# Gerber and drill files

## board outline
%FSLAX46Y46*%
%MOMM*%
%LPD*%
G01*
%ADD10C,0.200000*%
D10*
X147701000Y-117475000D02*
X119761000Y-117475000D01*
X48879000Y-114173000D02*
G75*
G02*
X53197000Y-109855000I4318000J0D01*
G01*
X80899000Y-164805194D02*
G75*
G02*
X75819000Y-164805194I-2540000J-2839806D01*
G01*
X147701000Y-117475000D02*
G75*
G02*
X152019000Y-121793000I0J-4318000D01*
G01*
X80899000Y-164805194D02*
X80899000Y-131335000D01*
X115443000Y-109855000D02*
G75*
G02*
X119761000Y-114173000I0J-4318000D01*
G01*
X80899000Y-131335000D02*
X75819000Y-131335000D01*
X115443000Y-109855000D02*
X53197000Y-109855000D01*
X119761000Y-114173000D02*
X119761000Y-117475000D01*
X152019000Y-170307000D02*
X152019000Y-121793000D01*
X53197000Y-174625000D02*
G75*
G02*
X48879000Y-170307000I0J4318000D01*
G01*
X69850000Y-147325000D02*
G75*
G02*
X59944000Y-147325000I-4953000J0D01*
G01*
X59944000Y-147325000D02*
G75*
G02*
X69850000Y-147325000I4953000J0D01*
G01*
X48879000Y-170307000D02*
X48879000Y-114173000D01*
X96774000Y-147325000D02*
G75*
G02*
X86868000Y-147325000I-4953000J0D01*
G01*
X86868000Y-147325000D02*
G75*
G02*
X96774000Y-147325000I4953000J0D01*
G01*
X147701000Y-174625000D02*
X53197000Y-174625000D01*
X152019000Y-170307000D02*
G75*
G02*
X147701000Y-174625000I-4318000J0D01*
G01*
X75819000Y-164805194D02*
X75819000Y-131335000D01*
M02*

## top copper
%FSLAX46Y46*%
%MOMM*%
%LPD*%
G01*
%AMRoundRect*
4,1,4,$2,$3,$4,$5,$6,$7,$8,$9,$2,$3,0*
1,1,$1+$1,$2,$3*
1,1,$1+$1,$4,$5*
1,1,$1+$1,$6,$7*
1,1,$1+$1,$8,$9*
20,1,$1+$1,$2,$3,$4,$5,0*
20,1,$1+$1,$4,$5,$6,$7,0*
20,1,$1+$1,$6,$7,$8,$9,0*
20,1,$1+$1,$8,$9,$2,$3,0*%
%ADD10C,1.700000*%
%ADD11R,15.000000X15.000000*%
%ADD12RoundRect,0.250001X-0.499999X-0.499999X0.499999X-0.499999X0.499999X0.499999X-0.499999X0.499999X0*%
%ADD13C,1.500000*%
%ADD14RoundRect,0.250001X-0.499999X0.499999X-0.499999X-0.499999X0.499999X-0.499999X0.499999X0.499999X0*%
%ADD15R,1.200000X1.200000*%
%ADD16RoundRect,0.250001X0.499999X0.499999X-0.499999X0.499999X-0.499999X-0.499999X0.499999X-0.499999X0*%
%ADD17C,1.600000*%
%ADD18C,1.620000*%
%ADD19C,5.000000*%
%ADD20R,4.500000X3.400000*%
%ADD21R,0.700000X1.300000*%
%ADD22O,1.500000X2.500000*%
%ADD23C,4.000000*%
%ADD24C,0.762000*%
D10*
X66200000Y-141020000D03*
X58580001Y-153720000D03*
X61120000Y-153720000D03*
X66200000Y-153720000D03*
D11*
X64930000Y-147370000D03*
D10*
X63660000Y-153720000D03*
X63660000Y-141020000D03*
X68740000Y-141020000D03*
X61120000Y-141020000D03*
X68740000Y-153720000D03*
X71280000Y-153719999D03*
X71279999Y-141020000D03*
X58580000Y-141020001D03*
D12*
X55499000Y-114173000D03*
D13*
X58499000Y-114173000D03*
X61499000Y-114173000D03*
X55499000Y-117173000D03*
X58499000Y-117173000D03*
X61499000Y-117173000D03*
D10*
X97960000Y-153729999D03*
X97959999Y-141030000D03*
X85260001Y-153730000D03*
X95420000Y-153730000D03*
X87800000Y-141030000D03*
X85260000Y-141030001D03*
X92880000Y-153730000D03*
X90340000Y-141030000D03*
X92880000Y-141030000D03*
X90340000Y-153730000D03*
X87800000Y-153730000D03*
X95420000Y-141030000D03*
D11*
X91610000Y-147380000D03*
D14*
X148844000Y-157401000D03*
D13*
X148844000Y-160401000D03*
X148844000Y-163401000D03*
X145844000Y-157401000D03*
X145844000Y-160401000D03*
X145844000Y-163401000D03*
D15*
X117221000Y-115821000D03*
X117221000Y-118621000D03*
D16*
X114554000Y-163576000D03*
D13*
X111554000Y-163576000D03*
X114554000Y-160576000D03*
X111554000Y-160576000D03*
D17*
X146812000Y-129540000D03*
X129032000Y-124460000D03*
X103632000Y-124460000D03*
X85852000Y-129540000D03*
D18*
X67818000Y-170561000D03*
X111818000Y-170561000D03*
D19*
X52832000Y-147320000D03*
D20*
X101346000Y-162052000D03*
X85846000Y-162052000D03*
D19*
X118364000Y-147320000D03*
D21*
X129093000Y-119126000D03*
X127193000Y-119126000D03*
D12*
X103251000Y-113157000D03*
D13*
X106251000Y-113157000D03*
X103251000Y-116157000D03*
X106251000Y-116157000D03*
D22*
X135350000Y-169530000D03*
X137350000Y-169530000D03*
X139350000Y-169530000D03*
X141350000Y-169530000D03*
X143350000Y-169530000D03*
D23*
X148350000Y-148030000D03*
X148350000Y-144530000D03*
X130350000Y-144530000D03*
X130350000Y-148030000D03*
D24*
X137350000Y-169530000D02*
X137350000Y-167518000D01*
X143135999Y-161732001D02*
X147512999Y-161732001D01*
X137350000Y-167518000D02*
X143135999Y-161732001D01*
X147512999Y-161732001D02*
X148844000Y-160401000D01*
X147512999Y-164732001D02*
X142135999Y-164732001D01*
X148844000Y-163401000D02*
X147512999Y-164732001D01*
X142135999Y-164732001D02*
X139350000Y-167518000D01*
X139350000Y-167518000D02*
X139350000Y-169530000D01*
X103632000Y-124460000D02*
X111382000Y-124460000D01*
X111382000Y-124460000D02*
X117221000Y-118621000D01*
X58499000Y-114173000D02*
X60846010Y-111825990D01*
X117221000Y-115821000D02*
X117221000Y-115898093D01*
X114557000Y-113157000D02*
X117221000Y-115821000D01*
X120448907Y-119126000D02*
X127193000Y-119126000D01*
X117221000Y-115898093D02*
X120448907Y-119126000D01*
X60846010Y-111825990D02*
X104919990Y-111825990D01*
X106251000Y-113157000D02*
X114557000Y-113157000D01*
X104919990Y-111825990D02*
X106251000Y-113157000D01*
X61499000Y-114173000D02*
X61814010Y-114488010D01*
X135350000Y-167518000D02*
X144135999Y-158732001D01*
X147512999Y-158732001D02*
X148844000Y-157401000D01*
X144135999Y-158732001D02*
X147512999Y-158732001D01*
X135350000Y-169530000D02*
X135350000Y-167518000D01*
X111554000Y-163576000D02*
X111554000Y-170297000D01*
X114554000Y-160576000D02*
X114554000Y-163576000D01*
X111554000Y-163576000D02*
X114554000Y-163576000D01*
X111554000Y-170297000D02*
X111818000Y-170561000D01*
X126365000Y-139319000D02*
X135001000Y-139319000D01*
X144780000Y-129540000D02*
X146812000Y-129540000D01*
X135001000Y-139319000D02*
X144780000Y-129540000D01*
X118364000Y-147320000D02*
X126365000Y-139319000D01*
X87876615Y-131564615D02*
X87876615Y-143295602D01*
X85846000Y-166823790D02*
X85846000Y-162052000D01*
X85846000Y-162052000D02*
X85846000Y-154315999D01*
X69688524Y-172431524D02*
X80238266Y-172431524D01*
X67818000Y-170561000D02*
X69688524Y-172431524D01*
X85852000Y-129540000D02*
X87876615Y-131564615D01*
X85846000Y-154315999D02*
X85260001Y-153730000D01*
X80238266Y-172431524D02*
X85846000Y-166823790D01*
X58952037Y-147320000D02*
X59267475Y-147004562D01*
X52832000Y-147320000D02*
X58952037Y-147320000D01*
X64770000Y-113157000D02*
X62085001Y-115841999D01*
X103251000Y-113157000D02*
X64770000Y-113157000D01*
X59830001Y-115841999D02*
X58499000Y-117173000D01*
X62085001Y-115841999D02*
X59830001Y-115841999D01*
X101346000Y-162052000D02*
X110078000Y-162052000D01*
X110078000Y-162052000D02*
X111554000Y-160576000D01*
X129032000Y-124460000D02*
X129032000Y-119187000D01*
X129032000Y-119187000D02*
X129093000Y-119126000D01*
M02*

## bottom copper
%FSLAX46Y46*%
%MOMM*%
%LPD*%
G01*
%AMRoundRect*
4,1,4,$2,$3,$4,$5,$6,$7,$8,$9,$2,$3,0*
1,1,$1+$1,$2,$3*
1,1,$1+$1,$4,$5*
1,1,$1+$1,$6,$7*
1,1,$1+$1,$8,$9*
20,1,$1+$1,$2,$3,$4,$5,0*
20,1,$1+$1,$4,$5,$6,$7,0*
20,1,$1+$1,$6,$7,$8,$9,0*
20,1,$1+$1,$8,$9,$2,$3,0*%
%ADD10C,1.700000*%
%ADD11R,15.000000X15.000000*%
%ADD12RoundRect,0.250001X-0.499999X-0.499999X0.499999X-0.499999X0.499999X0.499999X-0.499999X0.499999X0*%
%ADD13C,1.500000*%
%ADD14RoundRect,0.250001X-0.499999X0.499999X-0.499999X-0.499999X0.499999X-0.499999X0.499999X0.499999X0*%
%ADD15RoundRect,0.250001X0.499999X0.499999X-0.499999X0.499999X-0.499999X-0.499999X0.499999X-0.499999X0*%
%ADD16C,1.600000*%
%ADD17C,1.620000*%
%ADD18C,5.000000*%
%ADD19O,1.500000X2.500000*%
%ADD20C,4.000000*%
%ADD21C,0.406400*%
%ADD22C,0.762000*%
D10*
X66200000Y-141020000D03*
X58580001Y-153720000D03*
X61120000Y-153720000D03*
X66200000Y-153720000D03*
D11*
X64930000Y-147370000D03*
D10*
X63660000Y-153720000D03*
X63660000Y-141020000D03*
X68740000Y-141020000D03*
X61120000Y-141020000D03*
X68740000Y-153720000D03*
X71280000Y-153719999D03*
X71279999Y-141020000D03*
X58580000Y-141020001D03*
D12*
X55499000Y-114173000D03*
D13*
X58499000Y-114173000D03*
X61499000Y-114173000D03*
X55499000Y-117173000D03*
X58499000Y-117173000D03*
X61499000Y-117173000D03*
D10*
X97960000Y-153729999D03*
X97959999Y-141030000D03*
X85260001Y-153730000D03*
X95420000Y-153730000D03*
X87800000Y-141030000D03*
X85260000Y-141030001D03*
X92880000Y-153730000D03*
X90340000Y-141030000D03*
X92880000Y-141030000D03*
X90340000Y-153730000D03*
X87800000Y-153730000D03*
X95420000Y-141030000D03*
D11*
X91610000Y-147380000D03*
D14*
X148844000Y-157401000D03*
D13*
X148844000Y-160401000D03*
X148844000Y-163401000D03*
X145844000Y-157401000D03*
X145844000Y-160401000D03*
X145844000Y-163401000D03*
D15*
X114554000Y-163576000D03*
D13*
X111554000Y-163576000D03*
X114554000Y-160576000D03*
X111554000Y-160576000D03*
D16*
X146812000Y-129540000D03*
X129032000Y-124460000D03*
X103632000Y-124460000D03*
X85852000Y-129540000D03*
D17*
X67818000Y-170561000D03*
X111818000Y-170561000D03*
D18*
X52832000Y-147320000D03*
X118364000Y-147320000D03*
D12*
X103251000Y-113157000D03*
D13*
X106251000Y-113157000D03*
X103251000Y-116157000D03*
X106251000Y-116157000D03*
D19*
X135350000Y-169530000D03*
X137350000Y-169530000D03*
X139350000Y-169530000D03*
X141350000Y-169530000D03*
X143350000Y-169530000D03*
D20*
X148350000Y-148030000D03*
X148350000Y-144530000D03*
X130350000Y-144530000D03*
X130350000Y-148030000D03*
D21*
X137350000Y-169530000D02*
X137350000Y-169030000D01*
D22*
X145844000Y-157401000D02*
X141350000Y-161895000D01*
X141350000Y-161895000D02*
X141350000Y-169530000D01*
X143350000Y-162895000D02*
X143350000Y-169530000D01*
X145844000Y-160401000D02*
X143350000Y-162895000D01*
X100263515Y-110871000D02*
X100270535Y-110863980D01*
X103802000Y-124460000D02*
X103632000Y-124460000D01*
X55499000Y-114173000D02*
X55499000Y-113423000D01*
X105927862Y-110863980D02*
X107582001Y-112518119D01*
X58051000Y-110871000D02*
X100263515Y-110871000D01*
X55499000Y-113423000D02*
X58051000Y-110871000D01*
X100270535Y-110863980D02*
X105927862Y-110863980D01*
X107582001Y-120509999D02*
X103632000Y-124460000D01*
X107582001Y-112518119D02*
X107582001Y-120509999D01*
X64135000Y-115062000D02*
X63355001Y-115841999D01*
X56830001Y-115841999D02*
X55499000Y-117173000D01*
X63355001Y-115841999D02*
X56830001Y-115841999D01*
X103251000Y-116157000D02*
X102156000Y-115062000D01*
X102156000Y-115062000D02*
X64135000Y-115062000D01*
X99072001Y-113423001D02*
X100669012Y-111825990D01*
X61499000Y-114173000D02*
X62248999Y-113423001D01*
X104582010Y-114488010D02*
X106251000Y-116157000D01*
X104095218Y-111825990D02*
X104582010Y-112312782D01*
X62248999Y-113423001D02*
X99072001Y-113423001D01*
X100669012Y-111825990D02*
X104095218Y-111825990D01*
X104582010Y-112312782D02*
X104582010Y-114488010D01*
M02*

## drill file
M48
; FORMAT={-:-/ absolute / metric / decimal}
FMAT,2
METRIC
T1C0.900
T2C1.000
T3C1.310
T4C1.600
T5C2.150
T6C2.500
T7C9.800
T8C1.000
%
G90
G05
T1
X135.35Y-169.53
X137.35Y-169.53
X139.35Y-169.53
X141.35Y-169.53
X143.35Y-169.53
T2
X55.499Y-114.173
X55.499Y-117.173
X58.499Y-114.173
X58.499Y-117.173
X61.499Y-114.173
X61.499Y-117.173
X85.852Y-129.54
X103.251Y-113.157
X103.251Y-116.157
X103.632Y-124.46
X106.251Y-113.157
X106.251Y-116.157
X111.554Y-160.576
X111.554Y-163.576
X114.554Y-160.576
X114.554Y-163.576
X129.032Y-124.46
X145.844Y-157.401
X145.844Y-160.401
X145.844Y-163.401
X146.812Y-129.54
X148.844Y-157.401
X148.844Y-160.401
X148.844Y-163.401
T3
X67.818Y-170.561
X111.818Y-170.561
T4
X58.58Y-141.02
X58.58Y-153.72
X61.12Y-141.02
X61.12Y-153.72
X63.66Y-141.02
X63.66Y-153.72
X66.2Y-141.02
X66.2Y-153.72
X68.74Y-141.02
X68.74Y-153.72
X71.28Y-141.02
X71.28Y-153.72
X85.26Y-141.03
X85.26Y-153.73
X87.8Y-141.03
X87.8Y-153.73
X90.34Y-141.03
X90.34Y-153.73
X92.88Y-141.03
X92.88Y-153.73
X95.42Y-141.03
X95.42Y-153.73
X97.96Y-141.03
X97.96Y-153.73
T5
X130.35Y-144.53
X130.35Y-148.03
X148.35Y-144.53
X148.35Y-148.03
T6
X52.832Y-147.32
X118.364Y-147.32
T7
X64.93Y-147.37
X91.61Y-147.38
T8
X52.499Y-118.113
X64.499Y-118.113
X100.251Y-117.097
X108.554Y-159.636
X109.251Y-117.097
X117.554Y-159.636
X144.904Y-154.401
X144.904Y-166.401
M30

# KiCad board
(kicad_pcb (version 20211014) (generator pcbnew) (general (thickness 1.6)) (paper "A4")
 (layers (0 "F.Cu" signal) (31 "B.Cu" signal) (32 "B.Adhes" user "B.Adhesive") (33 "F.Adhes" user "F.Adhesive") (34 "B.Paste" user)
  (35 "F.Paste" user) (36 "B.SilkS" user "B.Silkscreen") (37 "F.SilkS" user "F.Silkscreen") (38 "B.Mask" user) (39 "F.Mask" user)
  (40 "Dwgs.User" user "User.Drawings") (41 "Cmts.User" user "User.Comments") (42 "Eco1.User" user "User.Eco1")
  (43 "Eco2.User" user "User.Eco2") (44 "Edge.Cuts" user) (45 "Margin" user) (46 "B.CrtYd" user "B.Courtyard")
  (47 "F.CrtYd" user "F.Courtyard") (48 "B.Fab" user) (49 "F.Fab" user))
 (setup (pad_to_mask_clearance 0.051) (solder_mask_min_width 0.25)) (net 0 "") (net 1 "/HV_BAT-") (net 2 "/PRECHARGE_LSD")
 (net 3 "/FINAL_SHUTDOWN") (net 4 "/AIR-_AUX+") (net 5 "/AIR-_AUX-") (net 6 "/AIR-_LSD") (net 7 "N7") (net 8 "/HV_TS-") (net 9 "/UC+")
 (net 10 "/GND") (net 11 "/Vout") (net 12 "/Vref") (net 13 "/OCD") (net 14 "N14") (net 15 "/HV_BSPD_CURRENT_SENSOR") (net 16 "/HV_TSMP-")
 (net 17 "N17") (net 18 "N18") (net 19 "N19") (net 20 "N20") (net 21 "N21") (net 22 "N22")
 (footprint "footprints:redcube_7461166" (layer "F.Cu") (at 64.93 147.37)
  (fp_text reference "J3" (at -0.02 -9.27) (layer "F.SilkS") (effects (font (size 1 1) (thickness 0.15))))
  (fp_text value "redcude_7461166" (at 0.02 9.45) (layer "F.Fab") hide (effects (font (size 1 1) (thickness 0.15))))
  (pad "1" thru_hole circle locked (at 1.27 -6.35) (size 1.7 1.7) (drill 1.6) (layers *.Cu *.Mask) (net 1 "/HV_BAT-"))
  (pad "1" thru_hole circle locked (at -6.349999 6.35) (size 1.7 1.7) (drill 1.6) (layers *.Cu *.Mask) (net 1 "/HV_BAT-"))
  (pad "1" thru_hole circle locked (at -3.81 6.35) (size 1.7 1.7) (drill 1.6) (layers *.Cu *.Mask) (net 1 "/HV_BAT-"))
  (pad "1" thru_hole circle locked (at 1.27 6.35) (size 1.7 1.7) (drill 1.6) (layers *.Cu *.Mask) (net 1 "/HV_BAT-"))
  (pad "1" thru_hole rect locked (at 0 0) (size 15 15) (drill 9.8) (layers *.Cu *.Mask) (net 1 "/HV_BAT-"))
  (pad "1" thru_hole circle locked (at -1.27 6.35) (size 1.7 1.7) (drill 1.6) (layers *.Cu *.Mask) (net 1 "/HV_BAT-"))
  (pad "1" thru_hole circle locked (at -1.27 -6.35) (size 1.7 1.7) (drill 1.6) (layers *.Cu *.Mask) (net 1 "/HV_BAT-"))
  (pad "1" thru_hole circle locked (at 3.81 -6.35) (size 1.7 1.7) (drill 1.6) (layers *.Cu *.Mask) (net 1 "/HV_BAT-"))
  (pad "1" thru_hole circle locked (at -3.81 -6.35) (size 1.7 1.7) (drill 1.6) (layers *.Cu *.Mask) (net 1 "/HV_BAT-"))
  (pad "1" thru_hole circle locked (at 3.81 6.35) (size 1.7 1.7) (drill 1.6) (layers *.Cu *.Mask) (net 1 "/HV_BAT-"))
  (pad "1" thru_hole circle locked (at 6.35 6.349999) (size 1.7 1.7) (drill 1.6) (layers *.Cu *.Mask) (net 1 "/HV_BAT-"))
  (pad "1" thru_hole circle locked (at 6.349999 -6.35) (size 1.7 1.7) (drill 1.6) (layers *.Cu *.Mask) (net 1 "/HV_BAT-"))
  (pad "1" thru_hole circle locked (at -6.35 -6.349999) (size 1.7 1.7) (drill 1.6) (layers *.Cu *.Mask) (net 1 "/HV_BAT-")))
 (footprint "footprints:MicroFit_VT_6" (layer "F.Cu") (at 55.499 114.173)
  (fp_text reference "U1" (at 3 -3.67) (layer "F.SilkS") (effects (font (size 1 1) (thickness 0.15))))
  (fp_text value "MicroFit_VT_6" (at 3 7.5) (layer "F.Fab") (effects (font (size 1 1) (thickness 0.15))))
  (pad "" np_thru_hole circle locked (at -3 3.94) (size 1 1) (drill 1) (layers *.Cu *.Mask))
  (pad "" np_thru_hole circle locked (at 9 3.94) (size 1 1) (drill 1) (layers *.Cu *.Mask))
  (pad "1" thru_hole roundrect locked (at 0 0) (size 1.5 1.5) (drill 1) (layers *.Cu *.Mask) (roundrect_rratio 0.166667)
   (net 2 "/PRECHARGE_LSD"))
  (pad "2" thru_hole circle locked (at 3 0) (size 1.5 1.5) (drill 1) (layers *.Cu *.Mask) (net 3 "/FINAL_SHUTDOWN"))
  (pad "3" thru_hole circle locked (at 6 0) (size 1.5 1.5) (drill 1) (layers *.Cu *.Mask) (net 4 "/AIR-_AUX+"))
  (pad "4" thru_hole circle locked (at 0 3) (size 1.5 1.5) (drill 1) (layers *.Cu *.Mask) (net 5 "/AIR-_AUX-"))
  (pad "5" thru_hole circle locked (at 3 3) (size 1.5 1.5) (drill 1) (layers *.Cu *.Mask) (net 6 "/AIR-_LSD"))
  (pad "6" thru_hole circle locked (at 6 3) (size 1.5 1.5) (drill 1) (layers *.Cu *.Mask) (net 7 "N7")))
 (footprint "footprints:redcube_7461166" (layer "F.Cu") (at 91.61 147.38)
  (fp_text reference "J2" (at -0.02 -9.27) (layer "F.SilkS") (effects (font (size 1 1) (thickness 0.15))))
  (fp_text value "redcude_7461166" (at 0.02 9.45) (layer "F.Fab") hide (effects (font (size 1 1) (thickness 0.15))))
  (pad "1" thru_hole circle locked (at 6.35 6.349999) (size 1.7 1.7) (drill 1.6) (layers *.Cu *.Mask) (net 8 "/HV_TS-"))
  (pad "1" thru_hole circle locked (at 6.349999 -6.35) (size 1.7 1.7) (drill 1.6) (layers *.Cu *.Mask) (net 8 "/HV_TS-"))
  (pad "1" thru_hole circle locked (at -6.349999 6.35) (size 1.7 1.7) (drill 1.6) (layers *.Cu *.Mask) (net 8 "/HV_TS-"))
  (pad "1" thru_hole circle locked (at 3.81 6.35) (size 1.7 1.7) (drill 1.6) (layers *.Cu *.Mask) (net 8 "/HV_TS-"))
  (pad "1" thru_hole circle locked (at -3.81 -6.35) (size 1.7 1.7) (drill 1.6) (layers *.Cu *.Mask) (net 8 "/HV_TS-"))
  (pad "1" thru_hole circle locked (at -6.35 -6.349999) (size 1.7 1.7) (drill 1.6) (layers *.Cu *.Mask) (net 8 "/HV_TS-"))
  (pad "1" thru_hole circle locked (at 1.27 6.35) (size 1.7 1.7) (drill 1.6) (layers *.Cu *.Mask) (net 8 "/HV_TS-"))
  (pad "1" thru_hole circle locked (at -1.27 -6.35) (size 1.7 1.7) (drill 1.6) (layers *.Cu *.Mask) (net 8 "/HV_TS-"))
  (pad "1" thru_hole circle locked (at 1.27 -6.35) (size 1.7 1.7) (drill 1.6) (layers *.Cu *.Mask) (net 8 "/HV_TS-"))
  (pad "1" thru_hole circle locked (at -1.27 6.35) (size 1.7 1.7) (drill 1.6) (layers *.Cu *.Mask) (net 8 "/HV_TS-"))
  (pad "1" thru_hole circle locked (at -3.81 6.35) (size 1.7 1.7) (drill 1.6) (layers *.Cu *.Mask) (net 8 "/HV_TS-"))
  (pad "1" thru_hole circle locked (at 3.81 -6.35) (size 1.7 1.7) (drill 1.6) (layers *.Cu *.Mask) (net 8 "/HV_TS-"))
  (pad "1" thru_hole rect locked (at 0 0) (size 15 15) (drill 9.8) (layers *.Cu *.Mask) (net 8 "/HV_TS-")))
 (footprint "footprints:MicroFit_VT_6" (layer "F.Cu") (at 148.844 157.401 -90)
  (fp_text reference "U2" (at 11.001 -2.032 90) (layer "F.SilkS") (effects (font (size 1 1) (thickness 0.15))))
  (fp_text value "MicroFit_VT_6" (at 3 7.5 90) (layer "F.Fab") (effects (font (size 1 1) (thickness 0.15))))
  (pad "" np_thru_hole circle locked (at 9 3.94 270) (size 1 1) (drill 1) (layers *.Cu *.Mask))
  (pad "" np_thru_hole circle locked (at -3 3.94 270) (size 1 1) (drill 1) (layers *.Cu *.Mask))
  (pad "1" thru_hole roundrect locked (at 0 0 270) (size 1.5 1.5) (drill 1) (layers *.Cu *.Mask) (roundrect_rratio 0.166667) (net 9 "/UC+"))
  (pad "2" thru_hole circle locked (at 3 0 270) (size 1.5 1.5) (drill 1) (layers *.Cu *.Mask) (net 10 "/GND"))
  (pad "3" thru_hole circle locked (at 6 0 270) (size 1.5 1.5) (drill 1) (layers *.Cu *.Mask) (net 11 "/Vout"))
  (pad "4" thru_hole circle locked (at 0 3 270) (size 1.5 1.5) (drill 1) (layers *.Cu *.Mask) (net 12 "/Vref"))
  (pad "5" thru_hole circle locked (at 3 3 270) (size 1.5 1.5) (drill 1) (layers *.Cu *.Mask) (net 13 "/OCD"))
  (pad "6" thru_hole circle locked (at 6 3 270) (size 1.5 1.5) (drill 1) (layers *.Cu *.Mask) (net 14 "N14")))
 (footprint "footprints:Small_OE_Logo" (layer "F.Cu") (at 60.071 127)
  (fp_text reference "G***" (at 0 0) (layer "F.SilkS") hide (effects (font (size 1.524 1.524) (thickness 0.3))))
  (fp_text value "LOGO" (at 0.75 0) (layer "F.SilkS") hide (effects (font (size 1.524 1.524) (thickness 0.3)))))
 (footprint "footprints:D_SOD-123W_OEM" (layer "F.Cu") (at 117.221 117.221 -90)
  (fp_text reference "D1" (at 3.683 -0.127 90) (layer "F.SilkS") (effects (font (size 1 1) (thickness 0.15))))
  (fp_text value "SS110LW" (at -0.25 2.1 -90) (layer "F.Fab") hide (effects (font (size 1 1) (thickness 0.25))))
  (pad "1" smd rect locked (at -1.4 0 270) (size 1.2 1.2) (layers "F.Cu" "F.Paste" "F.Mask") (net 3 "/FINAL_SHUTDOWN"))
  (pad "2" smd rect locked (at 1.4 0 270) (size 1.2 1.2) (layers "F.Cu" "F.Paste" "F.Mask") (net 2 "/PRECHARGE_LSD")))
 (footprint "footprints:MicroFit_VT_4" (layer "F.Cu") (at 114.554 163.576 180)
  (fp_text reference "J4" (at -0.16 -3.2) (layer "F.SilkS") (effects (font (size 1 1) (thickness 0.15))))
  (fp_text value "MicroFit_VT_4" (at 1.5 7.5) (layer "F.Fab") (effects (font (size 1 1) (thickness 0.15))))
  (pad "" np_thru_hole circle locked (at -3 3.94 180) (size 1 1) (drill 1) (layers *.Cu *.Mask))
  (pad "" np_thru_hole circle locked (at 6 3.94 180) (size 1 1) (drill 1) (layers *.Cu *.Mask))
  (pad "1" thru_hole roundrect locked (at 0 0 180) (size 1.5 1.5) (drill 1) (layers *.Cu *.Mask) (roundrect_rratio 0.166667)
   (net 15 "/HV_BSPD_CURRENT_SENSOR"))
  (pad "2" thru_hole circle locked (at 3 0 180) (size 1.5 1.5) (drill 1) (layers *.Cu *.Mask) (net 15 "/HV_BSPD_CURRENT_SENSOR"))
  (pad "3" thru_hole circle locked (at 0 3 180) (size 1.5 1.5) (drill 1) (layers *.Cu *.Mask) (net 15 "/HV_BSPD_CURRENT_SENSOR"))
  (pad "4" thru_hole circle locked (at 3 3 180) (size 1.5 1.5) (drill 1) (layers *.Cu *.Mask) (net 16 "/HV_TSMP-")))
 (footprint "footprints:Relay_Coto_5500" (layer "F.Cu") (at 82.042 137.033)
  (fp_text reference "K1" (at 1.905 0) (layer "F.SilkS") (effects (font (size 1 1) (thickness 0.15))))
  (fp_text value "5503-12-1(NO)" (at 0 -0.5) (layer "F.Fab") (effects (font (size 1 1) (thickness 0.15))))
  (pad "1" thru_hole circle locked (at 64.77 -7.493) (size 1.6 1.6) (drill 1) (layers *.Cu *.Mask) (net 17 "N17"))
  (pad "2" thru_hole circle locked (at 46.99 -12.573) (size 1.6 1.6) (drill 1) (layers *.Cu *.Mask) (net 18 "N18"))
  (pad "3" thru_hole circle locked (at 21.59 -12.573) (size 1.6 1.6) (drill 1) (layers *.Cu *.Mask) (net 2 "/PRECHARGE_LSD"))
  (pad "4" thru_hole circle locked (at 3.81 -7.493) (size 1.6 1.6) (drill 1) (layers *.Cu *.Mask) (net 8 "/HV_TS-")))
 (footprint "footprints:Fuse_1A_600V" (layer "F.Cu") (at 67.818 170.561)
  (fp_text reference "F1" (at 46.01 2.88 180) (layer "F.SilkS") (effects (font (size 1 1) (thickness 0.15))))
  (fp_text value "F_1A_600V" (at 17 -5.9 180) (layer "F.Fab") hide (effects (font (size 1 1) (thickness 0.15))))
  (pad "1" thru_hole circle locked (at 0 0) (size 1.62 1.62) (drill 1.31) (layers *.Cu *.Mask) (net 8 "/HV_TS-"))
  (pad "2" thru_hole circle locked (at 44 0) (size 1.62 1.62) (drill 1.31) (layers *.Cu *.Mask) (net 15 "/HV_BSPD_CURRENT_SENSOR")))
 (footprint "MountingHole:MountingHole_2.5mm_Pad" (layer "F.Cu") (at 52.832 147.32)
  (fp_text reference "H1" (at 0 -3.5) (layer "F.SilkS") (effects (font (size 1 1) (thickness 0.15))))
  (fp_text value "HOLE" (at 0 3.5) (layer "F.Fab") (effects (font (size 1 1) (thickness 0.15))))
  (pad "1" thru_hole circle locked (at 0 0) (size 5 5) (drill 2.5) (layers *.Cu *.Mask) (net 1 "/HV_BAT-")))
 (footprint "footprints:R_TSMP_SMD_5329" (layer "F.Cu") (at 93.726 162.052 180)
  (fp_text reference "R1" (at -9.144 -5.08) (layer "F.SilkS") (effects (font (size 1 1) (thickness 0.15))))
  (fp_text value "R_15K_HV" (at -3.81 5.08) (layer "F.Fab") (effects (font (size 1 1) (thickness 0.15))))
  (pad "1" smd rect locked (at -7.62 0 180) (size 4.5 3.4) (layers "F.Cu" "F.Paste" "F.Mask") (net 16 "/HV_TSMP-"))
  (pad "2" smd rect locked (at 7.88 0 180) (size 4.5 3.4) (layers "F.Cu" "F.Paste" "F.Mask") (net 8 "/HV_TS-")))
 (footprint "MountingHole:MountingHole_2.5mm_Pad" (layer "F.Cu") (at 118.364 147.32)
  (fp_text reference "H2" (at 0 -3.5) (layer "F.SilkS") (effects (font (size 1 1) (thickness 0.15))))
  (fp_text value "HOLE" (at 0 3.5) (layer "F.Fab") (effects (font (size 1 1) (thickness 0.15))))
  (pad "1" thru_hole circle locked (at 0 0) (size 5 5) (drill 2.5) (layers *.Cu *.Mask) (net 17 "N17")))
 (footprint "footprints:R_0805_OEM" (layer "F.Cu") (at 128.143 119.126 180)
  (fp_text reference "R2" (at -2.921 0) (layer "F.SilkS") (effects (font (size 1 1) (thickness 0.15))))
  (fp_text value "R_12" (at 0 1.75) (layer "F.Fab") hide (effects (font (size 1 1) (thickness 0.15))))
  (pad "1" smd rect locked (at -0.95 0 180) (size 0.7 1.3) (layers "F.Cu" "F.Paste" "F.Mask") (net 18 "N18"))
  (pad "2" smd rect locked (at 0.95 0 180) (size 0.7 1.3) (layers "F.Cu" "F.Paste" "F.Mask") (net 3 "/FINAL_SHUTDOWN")))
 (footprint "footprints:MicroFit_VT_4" (layer "F.Cu") (at 103.251 113.157)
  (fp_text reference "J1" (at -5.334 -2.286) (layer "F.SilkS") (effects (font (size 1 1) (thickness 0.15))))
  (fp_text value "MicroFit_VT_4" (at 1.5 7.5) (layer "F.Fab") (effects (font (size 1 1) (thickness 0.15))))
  (pad "" np_thru_hole circle locked (at 6 3.94) (size 1 1) (drill 1) (layers *.Cu *.Mask))
  (pad "" np_thru_hole circle locked (at -3 3.94) (size 1 1) (drill 1) (layers *.Cu *.Mask))
  (pad "1" thru_hole roundrect locked (at 0 0) (size 1.5 1.5) (drill 1) (layers *.Cu *.Mask) (roundrect_rratio 0.166667) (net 6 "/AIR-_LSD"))
  (pad "2" thru_hole circle locked (at 3 0) (size 1.5 1.5) (drill 1) (layers *.Cu *.Mask) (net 3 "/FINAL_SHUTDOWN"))
  (pad "3" thru_hole circle locked (at 0 3) (size 1.5 1.5) (drill 1) (layers *.Cu *.Mask) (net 5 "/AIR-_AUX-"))
  (pad "4" thru_hole circle locked (at 3 3) (size 1.5 1.5) (drill 1) (layers *.Cu *.Mask) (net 4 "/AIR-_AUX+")))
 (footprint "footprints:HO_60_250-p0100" (layer "B.Cu") (at 130.35 144.53 -90)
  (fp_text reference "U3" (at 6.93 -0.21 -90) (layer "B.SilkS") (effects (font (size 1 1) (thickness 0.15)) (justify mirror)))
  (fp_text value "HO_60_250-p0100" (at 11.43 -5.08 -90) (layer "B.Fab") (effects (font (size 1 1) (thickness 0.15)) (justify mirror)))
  (pad "1" thru_hole oval locked (at 25 -5 270) (size 2.5 1.5) (drill 0.9) (layers *.Cu *.Mask) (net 9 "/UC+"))
  (pad "2" thru_hole oval locked (at 25 -7 270) (size 2.5 1.5) (drill 0.9) (layers *.Cu *.Mask) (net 10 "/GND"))
  (pad "3" thru_hole oval locked (at 25 -9 270) (size 2.5 1.5) (drill 0.9) (layers *.Cu *.Mask) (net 11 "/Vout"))
  (pad "4" thru_hole oval locked (at 25 -11 270) (size 2.5 1.5) (drill 0.9) (layers *.Cu *.Mask) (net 12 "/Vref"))
  (pad "5" thru_hole oval locked (at 25 -13 270) (size 2.5 1.5) (drill 0.9) (layers *.Cu *.Mask) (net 13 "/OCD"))
  (pad "7" thru_hole circle locked (at 3.5 -18 270) (size 4 4) (drill 2.15) (layers *.Cu *.Mask) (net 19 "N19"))
  (pad "8" thru_hole circle locked (at 0 -18 270) (size 4 4) (drill 2.15) (layers *.Cu *.Mask) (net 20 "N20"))
  (pad "11" thru_hole circle locked (at 0 0 270) (size 4 4) (drill 2.15) (layers *.Cu *.Mask) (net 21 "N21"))
  (pad "12" thru_hole circle locked (at 3.5 0 270) (size 4 4) (drill 2.15) (layers *.Cu *.Mask) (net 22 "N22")))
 (gr_line (start 147.701 117.475) (end 119.761 117.475) (layer "Edge.Cuts") (width 0.2))
 (gr_arc (start 48.879 114.173) (mid 50.143713 111.119713) (end 53.197 109.855) (layer "Edge.Cuts") (width 0.2))
 (gr_arc (start 80.899 164.805194) (mid 78.359 171.455) (end 75.819 164.805194) (layer "Edge.Cuts") (width 0.2))
 (gr_arc (start 147.701 117.475) (mid 150.754287 118.739713) (end 152.019 121.793) (layer "Edge.Cuts") (width 0.2))
 (gr_line (start 80.899 164.805194) (end 80.899 131.335) (layer "Edge.Cuts") (width 0.2))
 (gr_arc (start 115.443 109.855) (mid 118.496287 111.119713) (end 119.761 114.173) (layer "Edge.Cuts") (width 0.2))
 (gr_line (start 80.899 131.335) (end 75.819 131.335) (layer "Edge.Cuts") (width 0.2))
 (gr_line (start 115.443 109.855) (end 53.197 109.855) (layer "Edge.Cuts") (width 0.2))
 (gr_line (start 119.761 114.173) (end 119.761 117.475) (layer "Edge.Cuts") (width 0.2))
 (gr_line (start 152.019 170.307) (end 152.019 121.793) (layer "Edge.Cuts") (width 0.2))
 (gr_arc (start 53.197 174.625) (mid 50.143713 173.360287) (end 48.879 170.307) (layer "Edge.Cuts") (width 0.2))
 (gr_circle (center 64.897 147.325) (end 59.944 147.325) (layer "Edge.Cuts") (width 0.2) (fill none))
 (gr_line (start 48.879 170.307) (end 48.879 114.173) (layer "Edge.Cuts") (width 0.2))
 (gr_circle (center 91.821 147.325) (end 86.868 147.325) (layer "Edge.Cuts") (width 0.2) (fill none))
 (gr_line (start 147.701 174.625) (end 53.197 174.625) (layer "Edge.Cuts") (width 0.2))
 (gr_arc (start 152.019 170.307) (mid 150.754287 173.360287) (end 147.701 174.625) (layer "Edge.Cuts") (width 0.2))
 (gr_line (start 75.819 164.805194) (end 75.819 131.335) (layer "Edge.Cuts") (width 0.2))
 (segment (start 137.35 169.53) (end 137.35 167.518) (width 0.762) (layer "F.Cu") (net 10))
 (segment (start 143.135999 161.732001) (end 147.512999 161.732001) (width 0.762) (layer "F.Cu") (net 10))
 (segment (start 137.35 167.518) (end 143.135999 161.732001) (width 0.762) (layer "F.Cu") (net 10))
 (segment (start 147.512999 161.732001) (end 148.844 160.401) (width 0.762) (layer "F.Cu") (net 10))
 (segment (start 137.35 169.53) (end 137.35 169.03) (width 0.4064) (layer "B.Cu") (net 10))
 (segment (start 147.512999 164.732001) (end 142.135999 164.732001) (width 0.762) (layer "F.Cu") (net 11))
 (segment (start 148.844 163.401) (end 147.512999 164.732001) (width 0.762) (layer "F.Cu") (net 11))
 (segment (start 142.135999 164.732001) (end 139.35 167.518) (width 0.762) (layer "F.Cu") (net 11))
 (segment (start 139.35 167.518) (end 139.35 169.53) (width 0.762) (layer "F.Cu") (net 11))
 (segment (start 145.844 157.401) (end 141.35 161.895) (width 0.762) (layer "B.Cu") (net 12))
 (segment (start 141.35 161.895) (end 141.35 169.53) (width 0.762) (layer "B.Cu") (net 12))
 (segment (start 143.35 162.895) (end 143.35 169.53) (width 0.762) (layer "B.Cu") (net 13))
 (segment (start 145.844 160.401) (end 143.35 162.895) (width 0.762) (layer "B.Cu") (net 13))
 (segment (start 103.632 124.46) (end 111.382 124.46) (width 0.762) (layer "F.Cu") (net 2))
 (segment (start 111.382 124.46) (end 117.221 118.621) (width 0.762) (layer "F.Cu") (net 2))
 (segment (start 100.263515 110.871) (end 100.270535 110.86398) (width 0.762) (layer "B.Cu") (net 2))
 (segment (start 103.802 124.46) (end 103.632 124.46) (width 0.762) (layer "B.Cu") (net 2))
 (segment (start 55.499 114.173) (end 55.499 113.423) (width 0.762) (layer "B.Cu") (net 2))
 (segment (start 105.927862 110.86398) (end 107.582001 112.518119) (width 0.762) (layer "B.Cu") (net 2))
 (segment (start 58.051 110.871) (end 100.263515 110.871) (width 0.762) (layer "B.Cu") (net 2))
 (segment (start 55.499 113.423) (end 58.051 110.871) (width 0.762) (layer "B.Cu") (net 2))
 (segment (start 100.270535 110.86398) (end 105.927862 110.86398) (width 0.762) (layer "B.Cu") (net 2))
 (segment (start 107.582001 120.509999) (end 103.632 124.46) (width 0.762) (layer "B.Cu") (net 2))
 (segment (start 107.582001 112.518119) (end 107.582001 120.509999) (width 0.762) (layer "B.Cu") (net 2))
 (segment (start 58.499 114.173) (end 60.84601 111.82599) (width 0.762) (layer "F.Cu") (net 3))
 (segment (start 117.221 115.821) (end 117.221 115.898093) (width 0.762) (layer "F.Cu") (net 3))
 (segment (start 114.557 113.157) (end 117.221 115.821) (width 0.762) (layer "F.Cu") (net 3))
 (segment (start 120.448907 119.126) (end 127.193 119.126) (width 0.762) (layer "F.Cu") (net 3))
 (segment (start 117.221 115.898093) (end 120.448907 119.126) (width 0.762) (layer "F.Cu") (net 3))
 (segment (start 60.84601 111.82599) (end 104.91999 111.82599) (width 0.762) (layer "F.Cu") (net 3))
 (segment (start 106.251 113.157) (end 114.557 113.157) (width 0.762) (layer "F.Cu") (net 3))
 (segment (start 104.91999 111.82599) (end 106.251 113.157) (width 0.762) (layer "F.Cu") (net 3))
 (segment (start 64.135 115.062) (end 63.355001 115.841999) (width 0.762) (layer "B.Cu") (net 5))
 (segment (start 56.830001 115.841999) (end 55.499 117.173) (width 0.762) (layer "B.Cu") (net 5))
 (segment (start 63.355001 115.841999) (end 56.830001 115.841999) (width 0.762) (layer "B.Cu") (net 5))
 (segment (start 103.251 116.157) (end 102.156 115.062) (width 0.762) (layer "B.Cu") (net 5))
 (segment (start 102.156 115.062) (end 64.135 115.062) (width 0.762) (layer "B.Cu") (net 5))
 (segment (start 61.499 114.173) (end 61.81401 114.48801) (width 0.762) (layer "F.Cu") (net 4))
 (segment (start 99.072001 113.423001) (end 100.669012 111.82599) (width 0.762) (layer "B.Cu") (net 4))
 (segment (start 61.499 114.173) (end 62.248999 113.423001) (width 0.762) (layer "B.Cu") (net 4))
 (segment (start 104.58201 114.48801) (end 106.251 116.157) (width 0.762) (layer "B.Cu") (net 4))
 (segment (start 104.095218 111.82599) (end 104.58201 112.312782) (width 0.762) (layer "B.Cu") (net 4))
 (segment (start 62.248999 113.423001) (end 99.072001 113.423001) (width 0.762) (layer "B.Cu") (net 4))
 (segment (start 100.669012 111.82599) (end 104.095218 111.82599) (width 0.762) (layer "B.Cu") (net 4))
 (segment (start 104.58201 112.312782) (end 104.58201 114.48801) (width 0.762) (layer "B.Cu") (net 4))
 (segment (start 135.35 167.518) (end 144.135999 158.732001) (width 0.762) (layer "F.Cu") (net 9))
 (segment (start 147.512999 158.732001) (end 148.844 157.401) (width 0.762) (layer "F.Cu") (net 9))
 (segment (start 144.135999 158.732001) (end 147.512999 158.732001) (width 0.762) (layer "F.Cu") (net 9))
 (segment (start 135.35 169.53) (end 135.35 167.518) (width 0.762) (layer "F.Cu") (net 9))
 (segment (start 111.554 163.576) (end 111.554 170.297) (width 0.762) (layer "F.Cu") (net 15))
 (segment (start 114.554 160.576) (end 114.554 163.576) (width 0.762) (layer "F.Cu") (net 15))
 (segment (start 111.554 163.576) (end 114.554 163.576) (width 0.762) (layer "F.Cu") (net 15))
 (segment (start 111.554 170.297) (end 111.818 170.561) (width 0.762) (layer "F.Cu") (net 15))
 (segment (start 126.365 139.319) (end 135.001 139.319) (width 0.762) (layer "F.Cu") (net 17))
 (segment (start 144.78 129.54) (end 146.812 129.54) (width 0.762) (layer "F.Cu") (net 17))
 (segment (start 135.001 139.319) (end 144.78 129.54) (width 0.762) (layer "F.Cu") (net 17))
 (segment (start 118.364 147.32) (end 126.365 139.319) (width 0.762) (layer "F.Cu") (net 17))
 (segment (start 87.876615 131.564615) (end 87.876615 143.295602) (width 0.762) (layer "F.Cu") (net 8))
 (segment (start 85.846 166.82379) (end 85.846 162.052) (width 0.762) (layer "F.Cu") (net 8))
 (segment (start 85.846 162.052) (end 85.846 154.315999) (width 0.762) (layer "F.Cu") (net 8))
 (segment (start 69.688524 172.431524) (end 80.238266 172.431524) (width 0.762) (layer "F.Cu") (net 8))
 (segment (start 67.818 170.561) (end 69.688524 172.431524) (width 0.762) (layer "F.Cu") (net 8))
 (segment (start 85.852 129.54) (end 87.876615 131.564615) (width 0.762) (layer "F.Cu") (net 8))
 (segment (start 85.846 154.315999) (end 85.260001 153.73) (width 0.762) (layer "F.Cu") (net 8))
 (segment (start 80.238266 172.431524) (end 85.846 166.82379) (width 0.762) (layer "F.Cu") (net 8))
 (segment (start 58.952037 147.32) (end 59.267475 147.004562) (width 0.762) (layer "F.Cu") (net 1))
 (segment (start 52.832 147.32) (end 58.952037 147.32) (width 0.762) (layer "F.Cu") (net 1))
 (segment (start 64.77 113.157) (end 62.085001 115.841999) (width 0.762) (layer "F.Cu") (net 6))
 (segment (start 103.251 113.157) (end 64.77 113.157) (width 0.762) (layer "F.Cu") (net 6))
 (segment (start 59.830001 115.841999) (end 58.499 117.173) (width 0.762) (layer "F.Cu") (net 6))
 (segment (start 62.085001 115.841999) (end 59.830001 115.841999) (width 0.762) (layer "F.Cu") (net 6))
 (segment (start 101.346 162.052) (end 110.078 162.052) (width 0.762) (layer "F.Cu") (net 16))
 (segment (start 110.078 162.052) (end 111.554 160.576) (width 0.762) (layer "F.Cu") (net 16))
 (segment (start 129.032 124.46) (end 129.032 119.187) (width 0.762) (layer "F.Cu") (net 18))
 (segment (start 129.032 119.187) (end 129.093 119.126) (width 0.762) (layer "F.Cu") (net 18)))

